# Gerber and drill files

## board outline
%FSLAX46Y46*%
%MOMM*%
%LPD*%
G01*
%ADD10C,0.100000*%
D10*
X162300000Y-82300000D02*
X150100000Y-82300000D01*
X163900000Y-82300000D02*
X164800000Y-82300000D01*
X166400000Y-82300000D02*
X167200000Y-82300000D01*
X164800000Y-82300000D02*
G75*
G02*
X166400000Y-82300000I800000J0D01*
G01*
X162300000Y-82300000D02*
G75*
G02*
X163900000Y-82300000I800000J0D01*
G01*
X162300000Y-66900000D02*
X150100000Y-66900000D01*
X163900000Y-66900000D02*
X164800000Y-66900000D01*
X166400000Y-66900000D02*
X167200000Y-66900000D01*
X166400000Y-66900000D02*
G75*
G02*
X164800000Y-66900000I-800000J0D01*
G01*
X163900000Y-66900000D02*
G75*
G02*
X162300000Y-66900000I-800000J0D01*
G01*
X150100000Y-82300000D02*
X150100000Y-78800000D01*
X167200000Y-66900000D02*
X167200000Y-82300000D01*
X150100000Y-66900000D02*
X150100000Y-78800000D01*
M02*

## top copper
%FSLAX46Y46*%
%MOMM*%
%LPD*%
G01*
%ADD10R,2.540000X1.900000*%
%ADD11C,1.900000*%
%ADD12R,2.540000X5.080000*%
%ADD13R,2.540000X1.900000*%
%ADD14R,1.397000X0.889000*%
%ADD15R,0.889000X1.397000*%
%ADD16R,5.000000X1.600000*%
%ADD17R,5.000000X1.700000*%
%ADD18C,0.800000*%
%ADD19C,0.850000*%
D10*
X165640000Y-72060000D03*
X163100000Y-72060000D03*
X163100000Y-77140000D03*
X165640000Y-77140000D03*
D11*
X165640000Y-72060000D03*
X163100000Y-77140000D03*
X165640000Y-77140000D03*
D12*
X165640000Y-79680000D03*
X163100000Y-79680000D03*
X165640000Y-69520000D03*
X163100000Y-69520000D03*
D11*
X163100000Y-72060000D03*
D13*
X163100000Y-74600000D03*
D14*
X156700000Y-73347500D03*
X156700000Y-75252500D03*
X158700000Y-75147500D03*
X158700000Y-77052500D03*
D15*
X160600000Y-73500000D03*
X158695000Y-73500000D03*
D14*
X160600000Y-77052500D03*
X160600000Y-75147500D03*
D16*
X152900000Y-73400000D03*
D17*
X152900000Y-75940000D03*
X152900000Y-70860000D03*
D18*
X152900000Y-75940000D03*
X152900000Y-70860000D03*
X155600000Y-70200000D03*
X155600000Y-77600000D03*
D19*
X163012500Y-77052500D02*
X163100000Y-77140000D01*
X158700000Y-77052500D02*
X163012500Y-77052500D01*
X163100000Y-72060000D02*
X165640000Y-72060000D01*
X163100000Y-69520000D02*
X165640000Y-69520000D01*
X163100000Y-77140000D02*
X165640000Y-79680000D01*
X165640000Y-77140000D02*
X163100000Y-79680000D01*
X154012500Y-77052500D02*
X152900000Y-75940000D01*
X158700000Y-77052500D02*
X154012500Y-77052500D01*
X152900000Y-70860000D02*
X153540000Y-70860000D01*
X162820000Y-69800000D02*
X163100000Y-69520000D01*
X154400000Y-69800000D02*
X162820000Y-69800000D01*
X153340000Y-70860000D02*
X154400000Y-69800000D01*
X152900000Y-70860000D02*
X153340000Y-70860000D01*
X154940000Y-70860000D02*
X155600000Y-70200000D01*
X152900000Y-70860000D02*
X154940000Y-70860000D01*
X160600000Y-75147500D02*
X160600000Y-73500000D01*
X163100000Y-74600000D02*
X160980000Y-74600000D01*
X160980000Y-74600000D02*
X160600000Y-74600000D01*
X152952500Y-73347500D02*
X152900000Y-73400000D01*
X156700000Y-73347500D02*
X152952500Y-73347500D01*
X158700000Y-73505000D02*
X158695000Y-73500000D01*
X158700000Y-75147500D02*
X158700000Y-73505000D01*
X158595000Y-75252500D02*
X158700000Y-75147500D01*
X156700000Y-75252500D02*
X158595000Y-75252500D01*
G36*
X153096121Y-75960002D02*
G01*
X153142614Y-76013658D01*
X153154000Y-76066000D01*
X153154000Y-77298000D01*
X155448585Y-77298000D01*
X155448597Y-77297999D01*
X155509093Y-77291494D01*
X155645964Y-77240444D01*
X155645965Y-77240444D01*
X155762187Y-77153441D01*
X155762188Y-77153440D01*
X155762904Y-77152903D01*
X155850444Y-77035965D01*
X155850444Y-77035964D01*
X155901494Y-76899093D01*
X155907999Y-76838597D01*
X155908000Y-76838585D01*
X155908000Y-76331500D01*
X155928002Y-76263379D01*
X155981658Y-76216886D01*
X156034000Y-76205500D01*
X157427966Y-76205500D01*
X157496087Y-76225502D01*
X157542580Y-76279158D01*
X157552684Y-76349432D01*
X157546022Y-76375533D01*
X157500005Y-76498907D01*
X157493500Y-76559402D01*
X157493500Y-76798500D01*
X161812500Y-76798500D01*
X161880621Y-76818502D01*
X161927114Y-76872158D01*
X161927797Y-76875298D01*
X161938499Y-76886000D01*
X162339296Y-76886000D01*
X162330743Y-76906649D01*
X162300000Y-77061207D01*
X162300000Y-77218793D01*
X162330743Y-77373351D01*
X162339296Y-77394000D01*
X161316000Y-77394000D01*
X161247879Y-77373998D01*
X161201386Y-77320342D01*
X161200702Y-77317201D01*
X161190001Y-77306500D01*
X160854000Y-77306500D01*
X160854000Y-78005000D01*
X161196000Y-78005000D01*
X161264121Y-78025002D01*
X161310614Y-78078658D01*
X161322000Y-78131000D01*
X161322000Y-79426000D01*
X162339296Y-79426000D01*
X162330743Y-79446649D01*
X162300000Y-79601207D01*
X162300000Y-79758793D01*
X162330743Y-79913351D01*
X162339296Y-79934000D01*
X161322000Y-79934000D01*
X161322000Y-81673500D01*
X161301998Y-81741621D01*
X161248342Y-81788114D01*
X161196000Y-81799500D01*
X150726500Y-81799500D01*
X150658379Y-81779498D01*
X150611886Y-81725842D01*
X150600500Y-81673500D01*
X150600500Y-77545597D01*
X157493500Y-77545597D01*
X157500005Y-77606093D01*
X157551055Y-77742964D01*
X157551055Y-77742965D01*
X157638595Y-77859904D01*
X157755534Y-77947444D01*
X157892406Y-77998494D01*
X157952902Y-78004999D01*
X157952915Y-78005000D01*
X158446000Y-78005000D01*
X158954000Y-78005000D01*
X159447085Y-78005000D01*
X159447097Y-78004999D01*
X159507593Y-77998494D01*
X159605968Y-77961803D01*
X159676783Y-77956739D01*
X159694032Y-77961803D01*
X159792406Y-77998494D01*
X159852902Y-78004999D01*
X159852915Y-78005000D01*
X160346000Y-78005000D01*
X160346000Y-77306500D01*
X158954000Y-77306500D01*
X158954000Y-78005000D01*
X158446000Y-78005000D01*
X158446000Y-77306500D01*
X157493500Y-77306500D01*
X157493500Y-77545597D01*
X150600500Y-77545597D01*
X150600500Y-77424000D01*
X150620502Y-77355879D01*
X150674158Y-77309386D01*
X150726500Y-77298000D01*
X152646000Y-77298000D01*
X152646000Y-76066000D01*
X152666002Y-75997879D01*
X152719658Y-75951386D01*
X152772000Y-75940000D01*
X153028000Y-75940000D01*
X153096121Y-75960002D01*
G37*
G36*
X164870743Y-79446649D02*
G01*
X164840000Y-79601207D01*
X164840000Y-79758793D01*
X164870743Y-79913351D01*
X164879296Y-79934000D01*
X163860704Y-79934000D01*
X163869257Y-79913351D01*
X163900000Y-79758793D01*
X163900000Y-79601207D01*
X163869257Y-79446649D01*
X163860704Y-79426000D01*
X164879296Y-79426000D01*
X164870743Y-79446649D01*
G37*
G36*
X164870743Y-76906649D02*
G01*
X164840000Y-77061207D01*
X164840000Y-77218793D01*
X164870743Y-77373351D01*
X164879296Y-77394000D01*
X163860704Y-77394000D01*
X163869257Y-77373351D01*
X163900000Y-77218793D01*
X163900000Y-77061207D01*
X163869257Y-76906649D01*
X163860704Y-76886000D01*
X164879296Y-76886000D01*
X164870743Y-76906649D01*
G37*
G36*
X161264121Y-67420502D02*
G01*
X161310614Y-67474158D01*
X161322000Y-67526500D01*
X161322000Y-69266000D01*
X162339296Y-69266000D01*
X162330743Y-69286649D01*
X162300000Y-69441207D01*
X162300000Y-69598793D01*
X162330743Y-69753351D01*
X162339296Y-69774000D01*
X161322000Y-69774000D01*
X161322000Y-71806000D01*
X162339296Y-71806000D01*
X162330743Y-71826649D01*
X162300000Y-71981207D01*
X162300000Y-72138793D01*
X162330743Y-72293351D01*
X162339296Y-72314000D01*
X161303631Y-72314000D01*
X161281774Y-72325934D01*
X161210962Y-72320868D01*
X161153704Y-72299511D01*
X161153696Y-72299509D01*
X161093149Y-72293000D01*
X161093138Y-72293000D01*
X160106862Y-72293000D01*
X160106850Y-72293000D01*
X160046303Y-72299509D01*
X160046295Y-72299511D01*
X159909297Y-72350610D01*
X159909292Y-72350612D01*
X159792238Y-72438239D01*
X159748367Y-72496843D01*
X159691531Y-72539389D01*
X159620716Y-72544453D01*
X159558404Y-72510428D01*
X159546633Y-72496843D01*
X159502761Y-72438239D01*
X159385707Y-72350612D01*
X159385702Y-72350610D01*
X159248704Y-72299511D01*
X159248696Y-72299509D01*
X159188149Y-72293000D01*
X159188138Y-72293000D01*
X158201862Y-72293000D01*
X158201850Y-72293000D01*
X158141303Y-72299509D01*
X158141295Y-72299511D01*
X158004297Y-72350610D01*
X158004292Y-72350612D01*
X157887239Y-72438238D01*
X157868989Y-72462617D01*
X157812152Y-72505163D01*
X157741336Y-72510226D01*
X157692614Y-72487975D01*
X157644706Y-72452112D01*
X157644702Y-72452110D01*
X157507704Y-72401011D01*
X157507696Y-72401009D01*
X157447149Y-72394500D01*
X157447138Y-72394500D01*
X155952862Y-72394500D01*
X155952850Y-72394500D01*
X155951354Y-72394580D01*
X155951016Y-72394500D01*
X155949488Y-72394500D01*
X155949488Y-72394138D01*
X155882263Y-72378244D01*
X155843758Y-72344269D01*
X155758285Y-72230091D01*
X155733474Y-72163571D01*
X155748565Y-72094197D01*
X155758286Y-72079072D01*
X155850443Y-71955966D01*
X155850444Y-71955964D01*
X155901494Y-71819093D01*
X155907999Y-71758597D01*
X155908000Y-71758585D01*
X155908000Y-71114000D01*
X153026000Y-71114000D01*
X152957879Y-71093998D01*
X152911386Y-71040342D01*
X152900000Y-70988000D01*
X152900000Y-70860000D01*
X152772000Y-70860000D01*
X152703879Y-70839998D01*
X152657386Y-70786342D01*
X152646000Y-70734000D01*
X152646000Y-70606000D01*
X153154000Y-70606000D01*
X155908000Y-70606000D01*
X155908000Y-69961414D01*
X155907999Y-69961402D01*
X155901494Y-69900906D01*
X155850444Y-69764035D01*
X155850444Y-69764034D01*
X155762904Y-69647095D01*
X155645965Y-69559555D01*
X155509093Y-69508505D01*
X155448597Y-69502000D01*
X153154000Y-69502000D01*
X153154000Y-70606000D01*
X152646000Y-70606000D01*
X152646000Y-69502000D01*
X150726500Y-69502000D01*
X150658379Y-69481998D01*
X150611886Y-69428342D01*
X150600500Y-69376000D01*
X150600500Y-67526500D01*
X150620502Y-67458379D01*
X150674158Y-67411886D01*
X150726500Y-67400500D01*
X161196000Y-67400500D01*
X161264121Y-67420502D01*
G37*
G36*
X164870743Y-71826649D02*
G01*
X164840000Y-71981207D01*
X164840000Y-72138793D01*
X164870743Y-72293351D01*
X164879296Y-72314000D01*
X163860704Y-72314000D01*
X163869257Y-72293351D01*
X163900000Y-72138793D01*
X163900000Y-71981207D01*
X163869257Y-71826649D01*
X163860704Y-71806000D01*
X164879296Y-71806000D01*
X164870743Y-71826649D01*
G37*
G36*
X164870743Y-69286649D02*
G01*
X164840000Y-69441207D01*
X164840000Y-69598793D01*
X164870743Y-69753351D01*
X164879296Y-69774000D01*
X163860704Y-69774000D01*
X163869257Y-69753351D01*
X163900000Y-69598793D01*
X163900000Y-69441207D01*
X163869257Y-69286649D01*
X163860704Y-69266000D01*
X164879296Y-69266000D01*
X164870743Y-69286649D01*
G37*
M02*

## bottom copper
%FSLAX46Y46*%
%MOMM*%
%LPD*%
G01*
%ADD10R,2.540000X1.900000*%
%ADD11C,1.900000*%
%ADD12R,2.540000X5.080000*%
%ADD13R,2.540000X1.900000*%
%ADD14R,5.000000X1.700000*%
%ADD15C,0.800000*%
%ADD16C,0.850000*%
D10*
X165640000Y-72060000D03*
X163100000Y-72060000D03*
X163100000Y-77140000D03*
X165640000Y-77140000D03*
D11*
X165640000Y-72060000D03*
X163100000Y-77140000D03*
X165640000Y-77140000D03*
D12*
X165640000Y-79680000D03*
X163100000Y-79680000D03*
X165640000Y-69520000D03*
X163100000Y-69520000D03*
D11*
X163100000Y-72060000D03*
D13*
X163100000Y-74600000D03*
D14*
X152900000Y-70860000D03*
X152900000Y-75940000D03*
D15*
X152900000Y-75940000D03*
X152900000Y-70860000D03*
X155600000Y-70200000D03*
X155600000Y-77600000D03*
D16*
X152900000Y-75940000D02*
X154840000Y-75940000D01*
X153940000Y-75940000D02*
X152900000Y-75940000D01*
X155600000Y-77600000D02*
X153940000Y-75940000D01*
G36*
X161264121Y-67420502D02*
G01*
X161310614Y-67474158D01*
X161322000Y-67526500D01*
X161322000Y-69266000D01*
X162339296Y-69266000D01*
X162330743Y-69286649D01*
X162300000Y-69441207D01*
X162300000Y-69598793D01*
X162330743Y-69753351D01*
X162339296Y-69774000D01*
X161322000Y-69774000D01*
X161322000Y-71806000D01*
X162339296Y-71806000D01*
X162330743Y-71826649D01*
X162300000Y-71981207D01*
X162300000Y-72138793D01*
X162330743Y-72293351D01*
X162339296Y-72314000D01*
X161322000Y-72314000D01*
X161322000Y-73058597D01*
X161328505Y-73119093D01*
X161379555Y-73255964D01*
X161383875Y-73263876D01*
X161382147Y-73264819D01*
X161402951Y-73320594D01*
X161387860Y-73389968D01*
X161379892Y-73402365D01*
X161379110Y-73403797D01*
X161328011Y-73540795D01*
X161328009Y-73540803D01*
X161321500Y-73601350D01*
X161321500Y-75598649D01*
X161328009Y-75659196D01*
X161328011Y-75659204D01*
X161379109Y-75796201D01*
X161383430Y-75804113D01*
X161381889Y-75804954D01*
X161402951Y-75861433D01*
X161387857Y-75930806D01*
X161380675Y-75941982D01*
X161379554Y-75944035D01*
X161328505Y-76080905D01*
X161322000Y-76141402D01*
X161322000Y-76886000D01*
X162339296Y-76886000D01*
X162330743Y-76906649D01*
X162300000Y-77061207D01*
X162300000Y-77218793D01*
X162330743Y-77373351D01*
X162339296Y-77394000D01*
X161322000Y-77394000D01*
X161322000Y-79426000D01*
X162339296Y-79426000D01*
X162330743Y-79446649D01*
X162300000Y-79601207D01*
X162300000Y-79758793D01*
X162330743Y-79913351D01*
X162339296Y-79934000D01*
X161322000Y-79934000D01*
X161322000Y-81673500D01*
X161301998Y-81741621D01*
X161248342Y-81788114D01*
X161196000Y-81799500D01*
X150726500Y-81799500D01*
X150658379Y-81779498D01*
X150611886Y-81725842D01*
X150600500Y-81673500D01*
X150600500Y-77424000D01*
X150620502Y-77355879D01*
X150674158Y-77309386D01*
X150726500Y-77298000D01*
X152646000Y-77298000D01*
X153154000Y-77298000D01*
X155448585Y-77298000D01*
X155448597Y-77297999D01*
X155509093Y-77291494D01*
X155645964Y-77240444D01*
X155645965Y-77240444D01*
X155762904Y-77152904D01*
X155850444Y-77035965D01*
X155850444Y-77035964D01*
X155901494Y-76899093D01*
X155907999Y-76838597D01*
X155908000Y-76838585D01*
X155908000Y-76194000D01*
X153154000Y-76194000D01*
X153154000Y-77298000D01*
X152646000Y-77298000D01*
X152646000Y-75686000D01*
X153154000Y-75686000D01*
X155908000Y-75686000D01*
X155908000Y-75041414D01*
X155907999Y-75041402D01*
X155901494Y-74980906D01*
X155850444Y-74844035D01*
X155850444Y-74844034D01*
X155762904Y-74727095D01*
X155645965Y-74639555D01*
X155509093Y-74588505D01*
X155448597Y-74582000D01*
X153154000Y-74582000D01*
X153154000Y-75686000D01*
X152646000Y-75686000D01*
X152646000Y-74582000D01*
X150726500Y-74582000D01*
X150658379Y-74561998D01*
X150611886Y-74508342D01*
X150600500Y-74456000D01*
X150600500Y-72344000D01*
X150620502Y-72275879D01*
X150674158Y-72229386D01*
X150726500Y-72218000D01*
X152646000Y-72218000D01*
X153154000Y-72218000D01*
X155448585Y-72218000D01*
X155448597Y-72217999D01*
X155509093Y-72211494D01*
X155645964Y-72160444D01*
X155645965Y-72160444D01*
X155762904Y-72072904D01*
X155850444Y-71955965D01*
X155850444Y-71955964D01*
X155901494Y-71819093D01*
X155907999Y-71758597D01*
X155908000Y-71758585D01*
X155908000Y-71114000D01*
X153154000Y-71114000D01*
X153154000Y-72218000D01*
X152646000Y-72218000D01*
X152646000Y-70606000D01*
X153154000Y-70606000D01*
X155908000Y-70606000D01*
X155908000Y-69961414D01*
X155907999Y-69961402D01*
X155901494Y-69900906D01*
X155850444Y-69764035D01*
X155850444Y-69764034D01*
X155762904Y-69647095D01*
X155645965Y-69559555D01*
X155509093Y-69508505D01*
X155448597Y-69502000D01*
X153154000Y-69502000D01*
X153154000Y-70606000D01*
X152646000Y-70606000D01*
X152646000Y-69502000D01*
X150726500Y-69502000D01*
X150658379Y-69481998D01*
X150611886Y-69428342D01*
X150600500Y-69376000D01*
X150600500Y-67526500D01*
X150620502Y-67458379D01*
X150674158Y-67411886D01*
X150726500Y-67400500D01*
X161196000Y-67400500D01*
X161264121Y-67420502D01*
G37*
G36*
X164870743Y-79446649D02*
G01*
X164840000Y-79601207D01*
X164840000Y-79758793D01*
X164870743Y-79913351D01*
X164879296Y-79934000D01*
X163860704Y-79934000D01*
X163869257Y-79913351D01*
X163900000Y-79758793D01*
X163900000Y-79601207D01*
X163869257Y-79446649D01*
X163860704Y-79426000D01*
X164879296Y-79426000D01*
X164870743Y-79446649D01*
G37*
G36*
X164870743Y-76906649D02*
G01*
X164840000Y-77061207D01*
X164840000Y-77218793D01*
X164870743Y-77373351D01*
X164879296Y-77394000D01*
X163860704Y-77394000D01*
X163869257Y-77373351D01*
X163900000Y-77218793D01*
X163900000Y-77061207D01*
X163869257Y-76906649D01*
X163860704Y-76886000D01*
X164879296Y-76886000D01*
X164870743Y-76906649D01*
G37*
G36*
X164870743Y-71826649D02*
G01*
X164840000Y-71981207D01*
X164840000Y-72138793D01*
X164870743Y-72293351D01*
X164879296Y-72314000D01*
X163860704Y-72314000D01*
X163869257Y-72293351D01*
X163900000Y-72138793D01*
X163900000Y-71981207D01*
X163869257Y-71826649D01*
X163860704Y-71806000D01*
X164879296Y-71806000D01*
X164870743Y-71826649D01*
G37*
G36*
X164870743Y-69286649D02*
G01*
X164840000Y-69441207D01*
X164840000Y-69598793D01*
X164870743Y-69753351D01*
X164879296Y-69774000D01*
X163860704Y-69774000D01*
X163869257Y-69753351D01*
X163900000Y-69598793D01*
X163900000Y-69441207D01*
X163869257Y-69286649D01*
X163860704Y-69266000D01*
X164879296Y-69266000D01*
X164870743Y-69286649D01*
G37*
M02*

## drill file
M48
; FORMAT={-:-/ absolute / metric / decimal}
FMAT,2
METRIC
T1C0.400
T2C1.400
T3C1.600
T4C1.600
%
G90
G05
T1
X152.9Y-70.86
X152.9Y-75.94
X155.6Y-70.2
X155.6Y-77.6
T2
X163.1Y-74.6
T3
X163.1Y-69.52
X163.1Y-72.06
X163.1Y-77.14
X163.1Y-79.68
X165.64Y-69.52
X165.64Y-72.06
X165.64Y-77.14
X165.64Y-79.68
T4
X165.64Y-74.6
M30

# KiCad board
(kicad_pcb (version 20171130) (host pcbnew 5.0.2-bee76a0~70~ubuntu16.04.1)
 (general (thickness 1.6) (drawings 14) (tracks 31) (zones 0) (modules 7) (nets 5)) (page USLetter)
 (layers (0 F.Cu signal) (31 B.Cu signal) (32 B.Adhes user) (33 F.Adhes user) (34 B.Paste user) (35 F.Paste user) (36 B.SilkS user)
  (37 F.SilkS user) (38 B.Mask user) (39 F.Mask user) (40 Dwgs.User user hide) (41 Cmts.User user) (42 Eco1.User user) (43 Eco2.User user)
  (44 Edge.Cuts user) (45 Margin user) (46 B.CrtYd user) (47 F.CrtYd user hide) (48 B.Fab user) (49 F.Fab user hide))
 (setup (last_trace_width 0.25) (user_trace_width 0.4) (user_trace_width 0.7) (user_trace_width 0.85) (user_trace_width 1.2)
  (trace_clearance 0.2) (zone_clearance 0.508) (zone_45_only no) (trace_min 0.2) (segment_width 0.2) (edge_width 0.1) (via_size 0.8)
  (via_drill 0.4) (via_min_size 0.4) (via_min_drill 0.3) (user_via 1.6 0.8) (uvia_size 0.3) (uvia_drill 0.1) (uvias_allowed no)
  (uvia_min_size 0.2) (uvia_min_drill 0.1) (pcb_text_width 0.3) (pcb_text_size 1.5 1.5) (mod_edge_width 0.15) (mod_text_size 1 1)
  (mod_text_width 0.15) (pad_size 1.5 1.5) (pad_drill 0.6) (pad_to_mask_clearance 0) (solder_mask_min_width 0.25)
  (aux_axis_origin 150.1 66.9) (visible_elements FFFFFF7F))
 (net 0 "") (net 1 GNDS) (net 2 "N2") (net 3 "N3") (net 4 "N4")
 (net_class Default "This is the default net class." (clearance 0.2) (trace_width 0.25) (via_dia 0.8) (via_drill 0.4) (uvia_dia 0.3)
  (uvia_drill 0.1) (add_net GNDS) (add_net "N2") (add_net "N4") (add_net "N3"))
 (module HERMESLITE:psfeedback (layer F.Cu) (at 163.1 74.6 270)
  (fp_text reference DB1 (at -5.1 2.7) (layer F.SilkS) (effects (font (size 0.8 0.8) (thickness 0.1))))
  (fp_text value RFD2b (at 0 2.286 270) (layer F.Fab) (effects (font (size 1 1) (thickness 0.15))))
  (pad 2 smd rect (at -2.54 -2.54 270) (size 1.9 2.54) (layers B.Cu B.Paste B.Mask) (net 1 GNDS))
  (pad 2 smd rect (at -2.54 0 270) (size 1.9 2.54) (layers B.Cu B.Paste B.Mask) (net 1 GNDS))
  (pad 2 smd rect (at 2.54 0 270) (size 1.9 2.54) (layers B.Cu B.Paste B.Mask) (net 1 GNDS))
  (pad 2 smd rect (at 2.54 -2.54 270) (size 1.9 2.54) (layers B.Cu B.Paste B.Mask) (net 1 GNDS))
  (pad 2 smd rect (at -2.54 -2.54 270) (size 1.9 2.54) (layers F.Cu F.Paste F.Mask) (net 1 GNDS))
  (pad 2 smd rect (at -2.54 0 270) (size 1.9 2.54) (layers F.Cu F.Paste F.Mask) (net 1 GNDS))
  (pad 2 smd rect (at 2.54 0 270) (size 1.9 2.54) (layers F.Cu F.Paste F.Mask) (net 1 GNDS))
  (pad 2 smd rect (at 2.54 -2.54 270) (size 1.9 2.54) (layers F.Cu F.Paste F.Mask) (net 1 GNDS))
  (pad 2 thru_hole circle (at -2.54 -2.54 270) (size 1.9 1.9) (drill 1.6) (layers *.Cu *.Mask) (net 1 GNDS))
  (pad "" np_thru_hole circle (at 0 -2.54 270) (size 1.6 1.6) (drill 1.6) (layers *.Cu *.Mask))
  (pad 2 thru_hole circle (at 2.54 0 270) (size 1.9 1.9) (drill 1.6) (layers *.Cu *.Mask) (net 1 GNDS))
  (pad 2 thru_hole circle (at 2.54 -2.54 270) (size 1.9 1.9) (drill 1.6) (layers *.Cu *.Mask) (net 1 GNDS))
  (pad 2 thru_hole rect (at 5.08 -2.54 270) (size 5.08 2.54) (drill 1.6) (layers *.Cu *.Mask) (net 1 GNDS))
  (pad 2 thru_hole rect (at 5.08 0 270) (size 5.08 2.54) (drill 1.6) (layers *.Cu *.Mask) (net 1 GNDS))
  (pad 2 thru_hole rect (at -5.08 -2.54 270) (size 5.08 2.54) (drill 1.6) (layers *.Cu *.Mask) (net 1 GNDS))
  (pad 2 thru_hole rect (at -5.08 0 270) (size 5.08 2.54) (drill 1.6) (layers *.Cu *.Mask) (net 1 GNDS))
  (pad 2 thru_hole circle (at -2.54 0 270) (size 1.9 1.9) (drill 1.6) (layers *.Cu *.Mask) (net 1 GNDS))
  (pad 1 thru_hole rect (at 0 0 270) (size 1.9 2.54) (drill 1.4) (layers *.Cu *.Mask) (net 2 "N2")))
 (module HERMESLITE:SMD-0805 (layer F.Cu) (at 156.7 74.3 90)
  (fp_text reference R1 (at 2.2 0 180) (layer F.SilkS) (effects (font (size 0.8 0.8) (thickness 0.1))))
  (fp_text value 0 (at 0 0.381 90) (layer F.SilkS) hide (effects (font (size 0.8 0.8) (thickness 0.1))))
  (pad 2 smd rect (at 0.9525 0 90) (size 0.889 1.397) (layers F.Cu F.Paste F.Mask) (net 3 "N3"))
  (pad 1 smd rect (at -0.9525 0 90) (size 0.889 1.397) (layers F.Cu F.Paste F.Mask) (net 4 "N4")))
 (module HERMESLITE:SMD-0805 (layer F.Cu) (at 158.7 76.1 270)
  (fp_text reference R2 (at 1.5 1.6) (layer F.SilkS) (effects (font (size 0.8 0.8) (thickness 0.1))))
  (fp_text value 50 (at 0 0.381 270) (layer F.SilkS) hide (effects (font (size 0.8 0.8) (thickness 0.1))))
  (pad 1 smd rect (at -0.9525 0 270) (size 0.889 1.397) (layers F.Cu F.Paste F.Mask) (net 4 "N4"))
  (pad 2 smd rect (at 0.9525 0 270) (size 0.889 1.397) (layers F.Cu F.Paste F.Mask) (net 1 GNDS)))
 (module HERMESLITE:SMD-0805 (layer F.Cu) (at 159.6475 73.5 180)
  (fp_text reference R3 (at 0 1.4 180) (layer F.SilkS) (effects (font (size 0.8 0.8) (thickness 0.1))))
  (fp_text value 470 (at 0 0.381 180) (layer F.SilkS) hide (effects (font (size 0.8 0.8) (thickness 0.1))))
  (pad 1 smd rect (at -0.9525 0 180) (size 0.889 1.397) (layers F.Cu F.Paste F.Mask) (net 2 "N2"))
  (pad 2 smd rect (at 0.9525 0 180) (size 0.889 1.397) (layers F.Cu F.Paste F.Mask) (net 4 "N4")))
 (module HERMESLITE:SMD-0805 (layer F.Cu) (at 160.6 76.1 270)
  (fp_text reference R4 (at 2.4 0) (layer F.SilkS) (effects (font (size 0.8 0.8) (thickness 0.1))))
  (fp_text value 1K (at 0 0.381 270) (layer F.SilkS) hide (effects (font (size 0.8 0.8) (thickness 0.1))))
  (pad 2 smd rect (at 0.9525 0 270) (size 0.889 1.397) (layers F.Cu F.Paste F.Mask) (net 1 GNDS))
  (pad 1 smd rect (at -0.9525 0 270) (size 0.889 1.397) (layers F.Cu F.Paste F.Mask) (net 2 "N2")))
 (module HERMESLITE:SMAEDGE (layer F.Cu) (at 155.6 73.4 90)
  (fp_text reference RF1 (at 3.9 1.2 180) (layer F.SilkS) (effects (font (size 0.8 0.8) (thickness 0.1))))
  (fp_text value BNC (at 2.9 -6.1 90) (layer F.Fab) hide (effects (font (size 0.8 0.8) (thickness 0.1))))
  (pad 1 smd rect (at 0 -2.7 90) (size 1.6 5) (layers F.Cu F.Paste F.Mask) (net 3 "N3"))
  (pad 2 smd rect (at -2.54 -2.7 90) (size 1.7 5) (layers F.Cu F.Paste F.Mask) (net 1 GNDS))
  (pad 2 smd rect (at 2.54 -2.7 90) (size 1.7 5) (layers F.Cu F.Paste F.Mask) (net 1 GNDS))
  (pad 2 smd rect (at 2.54 -2.7 90) (size 1.7 5) (layers *.Paste B.Cu B.Mask) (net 1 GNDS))
  (pad 2 smd rect (at -2.54 -2.7 90) (size 1.7 5) (layers B.Cu B.Paste B.Mask) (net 1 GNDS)))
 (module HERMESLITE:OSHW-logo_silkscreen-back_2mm (layer F.Cu) (at 160.3 80.3)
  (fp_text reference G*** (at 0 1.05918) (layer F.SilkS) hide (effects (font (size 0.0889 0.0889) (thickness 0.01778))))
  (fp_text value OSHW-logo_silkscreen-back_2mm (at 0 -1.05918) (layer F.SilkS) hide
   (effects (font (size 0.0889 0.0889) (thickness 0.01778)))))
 (gr_line (start 162.3 82.3) (end 150.1 82.3) (layer Edge.Cuts) (width 0.1))
 (gr_line (start 163.9 82.3) (end 164.8 82.3) (layer Edge.Cuts) (width 0.1))
 (gr_line (start 166.4 82.3) (end 167.2 82.3) (layer Edge.Cuts) (width 0.1))
 (gr_arc (start 165.6 82.3) (end 166.4 82.3) (angle -180) (layer Edge.Cuts) (width 0.1))
 (gr_arc (start 163.1 82.3) (end 163.9 82.3) (angle -180) (layer Edge.Cuts) (width 0.1))
 (gr_line (start 162.3 66.9) (end 150.1 66.9) (layer Edge.Cuts) (width 0.1))
 (gr_line (start 163.9 66.9) (end 164.8 66.9) (layer Edge.Cuts) (width 0.1))
 (gr_line (start 166.4 66.9) (end 167.2 66.9) (layer Edge.Cuts) (width 0.1))
 (gr_arc (start 165.6 66.9) (end 164.8 66.9) (angle -180) (layer Edge.Cuts) (width 0.1))
 (gr_arc (start 163.1 66.9) (end 162.3 66.9) (angle -180) (layer Edge.Cuts) (width 0.1))
 (gr_line (start 150.1 82.3) (end 150.1 78.8) (layer Edge.Cuts) (width 0.1))
 (gr_line (start 167.2 66.9) (end 167.2 82.3) (layer Edge.Cuts) (width 0.1))
 (gr_line (start 150.1 66.9) (end 150.1 78.8) (layer Edge.Cuts) (width 0.1))
 (segment (start 163.0125 77.0525) (end 163.1 77.14) (width 0.85) (layer F.Cu) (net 1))
 (segment (start 158.7 77.0525) (end 163.0125 77.0525) (width 0.85) (layer F.Cu) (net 1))
 (segment (start 163.1 72.06) (end 165.64 72.06) (width 0.85) (layer F.Cu) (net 1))
 (segment (start 163.1 69.52) (end 165.64 69.52) (width 0.85) (layer F.Cu) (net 1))
 (segment (start 163.1 77.14) (end 165.64 79.68) (width 0.85) (layer F.Cu) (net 1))
 (segment (start 165.64 77.14) (end 163.1 79.68) (width 0.85) (layer F.Cu) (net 1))
 (segment (start 154.0125 77.0525) (end 152.9 75.94) (width 0.85) (layer F.Cu) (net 1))
 (segment (start 158.7 77.0525) (end 154.0125 77.0525) (width 0.85) (layer F.Cu) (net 1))
 (segment (start 152.9 70.86) (end 153.54 70.86) (width 0.85) (layer F.Cu) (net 1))
 (segment (start 162.82 69.8) (end 163.1 69.52) (width 0.85) (layer F.Cu) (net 1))
 (segment (start 154.4 69.8) (end 162.82 69.8) (width 0.85) (layer F.Cu) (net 1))
 (segment (start 153.34 70.86) (end 154.4 69.8) (width 0.85) (layer F.Cu) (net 1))
 (segment (start 152.9 70.86) (end 153.34 70.86) (width 0.85) (layer F.Cu) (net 1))
 (via (at 152.9 75.94) (size 0.8) (drill 0.4) (layers F.Cu B.Cu) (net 1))
 (via (at 152.9 70.86) (size 0.8) (drill 0.4) (layers F.Cu B.Cu) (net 1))
 (via (at 155.6 70.2) (size 0.8) (drill 0.4) (layers F.Cu B.Cu) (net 1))
 (segment (start 154.94 70.86) (end 155.6 70.2) (width 0.85) (layer F.Cu) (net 1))
 (segment (start 152.9 70.86) (end 154.94 70.86) (width 0.85) (layer F.Cu) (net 1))
 (segment (start 152.9 75.94) (end 154.84 75.94) (width 0.85) (layer B.Cu) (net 1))
 (via (at 155.6 77.6) (size 0.8) (drill 0.4) (layers F.Cu B.Cu) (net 1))
 (segment (start 153.94 75.94) (end 152.9 75.94) (width 0.85) (layer B.Cu) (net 1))
 (segment (start 155.6 77.6) (end 153.94 75.94) (width 0.85) (layer B.Cu) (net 1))
 (segment (start 160.6 75.1475) (end 160.6 73.5) (width 0.85) (layer F.Cu) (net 2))
 (segment (start 163.1 74.6) (end 160.98 74.6) (width 0.85) (layer F.Cu) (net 2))
 (segment (start 160.98 74.6) (end 160.6 74.6) (width 0.85) (layer F.Cu) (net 2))
 (segment (start 152.9525 73.3475) (end 152.9 73.4) (width 0.85) (layer F.Cu) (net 3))
 (segment (start 156.7 73.3475) (end 152.9525 73.3475) (width 0.85) (layer F.Cu) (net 3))
 (segment (start 158.7 73.505) (end 158.695 73.5) (width 0.85) (layer F.Cu) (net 4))
 (segment (start 158.7 75.1475) (end 158.7 73.505) (width 0.85) (layer F.Cu) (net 4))
 (segment (start 158.595 75.2525) (end 158.7 75.1475) (width 0.85) (layer F.Cu) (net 4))
 (segment (start 156.7 75.2525) (end 158.595 75.2525) (width 0.85) (layer F.Cu) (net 4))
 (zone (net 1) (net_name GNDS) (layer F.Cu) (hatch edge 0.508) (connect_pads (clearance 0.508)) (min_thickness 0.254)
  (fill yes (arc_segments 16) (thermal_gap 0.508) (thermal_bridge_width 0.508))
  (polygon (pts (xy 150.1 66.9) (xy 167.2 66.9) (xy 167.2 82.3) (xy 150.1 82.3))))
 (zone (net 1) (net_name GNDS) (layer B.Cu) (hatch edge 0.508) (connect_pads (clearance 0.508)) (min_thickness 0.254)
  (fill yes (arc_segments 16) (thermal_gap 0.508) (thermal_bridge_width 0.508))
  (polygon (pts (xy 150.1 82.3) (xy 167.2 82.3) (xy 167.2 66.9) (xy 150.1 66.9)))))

